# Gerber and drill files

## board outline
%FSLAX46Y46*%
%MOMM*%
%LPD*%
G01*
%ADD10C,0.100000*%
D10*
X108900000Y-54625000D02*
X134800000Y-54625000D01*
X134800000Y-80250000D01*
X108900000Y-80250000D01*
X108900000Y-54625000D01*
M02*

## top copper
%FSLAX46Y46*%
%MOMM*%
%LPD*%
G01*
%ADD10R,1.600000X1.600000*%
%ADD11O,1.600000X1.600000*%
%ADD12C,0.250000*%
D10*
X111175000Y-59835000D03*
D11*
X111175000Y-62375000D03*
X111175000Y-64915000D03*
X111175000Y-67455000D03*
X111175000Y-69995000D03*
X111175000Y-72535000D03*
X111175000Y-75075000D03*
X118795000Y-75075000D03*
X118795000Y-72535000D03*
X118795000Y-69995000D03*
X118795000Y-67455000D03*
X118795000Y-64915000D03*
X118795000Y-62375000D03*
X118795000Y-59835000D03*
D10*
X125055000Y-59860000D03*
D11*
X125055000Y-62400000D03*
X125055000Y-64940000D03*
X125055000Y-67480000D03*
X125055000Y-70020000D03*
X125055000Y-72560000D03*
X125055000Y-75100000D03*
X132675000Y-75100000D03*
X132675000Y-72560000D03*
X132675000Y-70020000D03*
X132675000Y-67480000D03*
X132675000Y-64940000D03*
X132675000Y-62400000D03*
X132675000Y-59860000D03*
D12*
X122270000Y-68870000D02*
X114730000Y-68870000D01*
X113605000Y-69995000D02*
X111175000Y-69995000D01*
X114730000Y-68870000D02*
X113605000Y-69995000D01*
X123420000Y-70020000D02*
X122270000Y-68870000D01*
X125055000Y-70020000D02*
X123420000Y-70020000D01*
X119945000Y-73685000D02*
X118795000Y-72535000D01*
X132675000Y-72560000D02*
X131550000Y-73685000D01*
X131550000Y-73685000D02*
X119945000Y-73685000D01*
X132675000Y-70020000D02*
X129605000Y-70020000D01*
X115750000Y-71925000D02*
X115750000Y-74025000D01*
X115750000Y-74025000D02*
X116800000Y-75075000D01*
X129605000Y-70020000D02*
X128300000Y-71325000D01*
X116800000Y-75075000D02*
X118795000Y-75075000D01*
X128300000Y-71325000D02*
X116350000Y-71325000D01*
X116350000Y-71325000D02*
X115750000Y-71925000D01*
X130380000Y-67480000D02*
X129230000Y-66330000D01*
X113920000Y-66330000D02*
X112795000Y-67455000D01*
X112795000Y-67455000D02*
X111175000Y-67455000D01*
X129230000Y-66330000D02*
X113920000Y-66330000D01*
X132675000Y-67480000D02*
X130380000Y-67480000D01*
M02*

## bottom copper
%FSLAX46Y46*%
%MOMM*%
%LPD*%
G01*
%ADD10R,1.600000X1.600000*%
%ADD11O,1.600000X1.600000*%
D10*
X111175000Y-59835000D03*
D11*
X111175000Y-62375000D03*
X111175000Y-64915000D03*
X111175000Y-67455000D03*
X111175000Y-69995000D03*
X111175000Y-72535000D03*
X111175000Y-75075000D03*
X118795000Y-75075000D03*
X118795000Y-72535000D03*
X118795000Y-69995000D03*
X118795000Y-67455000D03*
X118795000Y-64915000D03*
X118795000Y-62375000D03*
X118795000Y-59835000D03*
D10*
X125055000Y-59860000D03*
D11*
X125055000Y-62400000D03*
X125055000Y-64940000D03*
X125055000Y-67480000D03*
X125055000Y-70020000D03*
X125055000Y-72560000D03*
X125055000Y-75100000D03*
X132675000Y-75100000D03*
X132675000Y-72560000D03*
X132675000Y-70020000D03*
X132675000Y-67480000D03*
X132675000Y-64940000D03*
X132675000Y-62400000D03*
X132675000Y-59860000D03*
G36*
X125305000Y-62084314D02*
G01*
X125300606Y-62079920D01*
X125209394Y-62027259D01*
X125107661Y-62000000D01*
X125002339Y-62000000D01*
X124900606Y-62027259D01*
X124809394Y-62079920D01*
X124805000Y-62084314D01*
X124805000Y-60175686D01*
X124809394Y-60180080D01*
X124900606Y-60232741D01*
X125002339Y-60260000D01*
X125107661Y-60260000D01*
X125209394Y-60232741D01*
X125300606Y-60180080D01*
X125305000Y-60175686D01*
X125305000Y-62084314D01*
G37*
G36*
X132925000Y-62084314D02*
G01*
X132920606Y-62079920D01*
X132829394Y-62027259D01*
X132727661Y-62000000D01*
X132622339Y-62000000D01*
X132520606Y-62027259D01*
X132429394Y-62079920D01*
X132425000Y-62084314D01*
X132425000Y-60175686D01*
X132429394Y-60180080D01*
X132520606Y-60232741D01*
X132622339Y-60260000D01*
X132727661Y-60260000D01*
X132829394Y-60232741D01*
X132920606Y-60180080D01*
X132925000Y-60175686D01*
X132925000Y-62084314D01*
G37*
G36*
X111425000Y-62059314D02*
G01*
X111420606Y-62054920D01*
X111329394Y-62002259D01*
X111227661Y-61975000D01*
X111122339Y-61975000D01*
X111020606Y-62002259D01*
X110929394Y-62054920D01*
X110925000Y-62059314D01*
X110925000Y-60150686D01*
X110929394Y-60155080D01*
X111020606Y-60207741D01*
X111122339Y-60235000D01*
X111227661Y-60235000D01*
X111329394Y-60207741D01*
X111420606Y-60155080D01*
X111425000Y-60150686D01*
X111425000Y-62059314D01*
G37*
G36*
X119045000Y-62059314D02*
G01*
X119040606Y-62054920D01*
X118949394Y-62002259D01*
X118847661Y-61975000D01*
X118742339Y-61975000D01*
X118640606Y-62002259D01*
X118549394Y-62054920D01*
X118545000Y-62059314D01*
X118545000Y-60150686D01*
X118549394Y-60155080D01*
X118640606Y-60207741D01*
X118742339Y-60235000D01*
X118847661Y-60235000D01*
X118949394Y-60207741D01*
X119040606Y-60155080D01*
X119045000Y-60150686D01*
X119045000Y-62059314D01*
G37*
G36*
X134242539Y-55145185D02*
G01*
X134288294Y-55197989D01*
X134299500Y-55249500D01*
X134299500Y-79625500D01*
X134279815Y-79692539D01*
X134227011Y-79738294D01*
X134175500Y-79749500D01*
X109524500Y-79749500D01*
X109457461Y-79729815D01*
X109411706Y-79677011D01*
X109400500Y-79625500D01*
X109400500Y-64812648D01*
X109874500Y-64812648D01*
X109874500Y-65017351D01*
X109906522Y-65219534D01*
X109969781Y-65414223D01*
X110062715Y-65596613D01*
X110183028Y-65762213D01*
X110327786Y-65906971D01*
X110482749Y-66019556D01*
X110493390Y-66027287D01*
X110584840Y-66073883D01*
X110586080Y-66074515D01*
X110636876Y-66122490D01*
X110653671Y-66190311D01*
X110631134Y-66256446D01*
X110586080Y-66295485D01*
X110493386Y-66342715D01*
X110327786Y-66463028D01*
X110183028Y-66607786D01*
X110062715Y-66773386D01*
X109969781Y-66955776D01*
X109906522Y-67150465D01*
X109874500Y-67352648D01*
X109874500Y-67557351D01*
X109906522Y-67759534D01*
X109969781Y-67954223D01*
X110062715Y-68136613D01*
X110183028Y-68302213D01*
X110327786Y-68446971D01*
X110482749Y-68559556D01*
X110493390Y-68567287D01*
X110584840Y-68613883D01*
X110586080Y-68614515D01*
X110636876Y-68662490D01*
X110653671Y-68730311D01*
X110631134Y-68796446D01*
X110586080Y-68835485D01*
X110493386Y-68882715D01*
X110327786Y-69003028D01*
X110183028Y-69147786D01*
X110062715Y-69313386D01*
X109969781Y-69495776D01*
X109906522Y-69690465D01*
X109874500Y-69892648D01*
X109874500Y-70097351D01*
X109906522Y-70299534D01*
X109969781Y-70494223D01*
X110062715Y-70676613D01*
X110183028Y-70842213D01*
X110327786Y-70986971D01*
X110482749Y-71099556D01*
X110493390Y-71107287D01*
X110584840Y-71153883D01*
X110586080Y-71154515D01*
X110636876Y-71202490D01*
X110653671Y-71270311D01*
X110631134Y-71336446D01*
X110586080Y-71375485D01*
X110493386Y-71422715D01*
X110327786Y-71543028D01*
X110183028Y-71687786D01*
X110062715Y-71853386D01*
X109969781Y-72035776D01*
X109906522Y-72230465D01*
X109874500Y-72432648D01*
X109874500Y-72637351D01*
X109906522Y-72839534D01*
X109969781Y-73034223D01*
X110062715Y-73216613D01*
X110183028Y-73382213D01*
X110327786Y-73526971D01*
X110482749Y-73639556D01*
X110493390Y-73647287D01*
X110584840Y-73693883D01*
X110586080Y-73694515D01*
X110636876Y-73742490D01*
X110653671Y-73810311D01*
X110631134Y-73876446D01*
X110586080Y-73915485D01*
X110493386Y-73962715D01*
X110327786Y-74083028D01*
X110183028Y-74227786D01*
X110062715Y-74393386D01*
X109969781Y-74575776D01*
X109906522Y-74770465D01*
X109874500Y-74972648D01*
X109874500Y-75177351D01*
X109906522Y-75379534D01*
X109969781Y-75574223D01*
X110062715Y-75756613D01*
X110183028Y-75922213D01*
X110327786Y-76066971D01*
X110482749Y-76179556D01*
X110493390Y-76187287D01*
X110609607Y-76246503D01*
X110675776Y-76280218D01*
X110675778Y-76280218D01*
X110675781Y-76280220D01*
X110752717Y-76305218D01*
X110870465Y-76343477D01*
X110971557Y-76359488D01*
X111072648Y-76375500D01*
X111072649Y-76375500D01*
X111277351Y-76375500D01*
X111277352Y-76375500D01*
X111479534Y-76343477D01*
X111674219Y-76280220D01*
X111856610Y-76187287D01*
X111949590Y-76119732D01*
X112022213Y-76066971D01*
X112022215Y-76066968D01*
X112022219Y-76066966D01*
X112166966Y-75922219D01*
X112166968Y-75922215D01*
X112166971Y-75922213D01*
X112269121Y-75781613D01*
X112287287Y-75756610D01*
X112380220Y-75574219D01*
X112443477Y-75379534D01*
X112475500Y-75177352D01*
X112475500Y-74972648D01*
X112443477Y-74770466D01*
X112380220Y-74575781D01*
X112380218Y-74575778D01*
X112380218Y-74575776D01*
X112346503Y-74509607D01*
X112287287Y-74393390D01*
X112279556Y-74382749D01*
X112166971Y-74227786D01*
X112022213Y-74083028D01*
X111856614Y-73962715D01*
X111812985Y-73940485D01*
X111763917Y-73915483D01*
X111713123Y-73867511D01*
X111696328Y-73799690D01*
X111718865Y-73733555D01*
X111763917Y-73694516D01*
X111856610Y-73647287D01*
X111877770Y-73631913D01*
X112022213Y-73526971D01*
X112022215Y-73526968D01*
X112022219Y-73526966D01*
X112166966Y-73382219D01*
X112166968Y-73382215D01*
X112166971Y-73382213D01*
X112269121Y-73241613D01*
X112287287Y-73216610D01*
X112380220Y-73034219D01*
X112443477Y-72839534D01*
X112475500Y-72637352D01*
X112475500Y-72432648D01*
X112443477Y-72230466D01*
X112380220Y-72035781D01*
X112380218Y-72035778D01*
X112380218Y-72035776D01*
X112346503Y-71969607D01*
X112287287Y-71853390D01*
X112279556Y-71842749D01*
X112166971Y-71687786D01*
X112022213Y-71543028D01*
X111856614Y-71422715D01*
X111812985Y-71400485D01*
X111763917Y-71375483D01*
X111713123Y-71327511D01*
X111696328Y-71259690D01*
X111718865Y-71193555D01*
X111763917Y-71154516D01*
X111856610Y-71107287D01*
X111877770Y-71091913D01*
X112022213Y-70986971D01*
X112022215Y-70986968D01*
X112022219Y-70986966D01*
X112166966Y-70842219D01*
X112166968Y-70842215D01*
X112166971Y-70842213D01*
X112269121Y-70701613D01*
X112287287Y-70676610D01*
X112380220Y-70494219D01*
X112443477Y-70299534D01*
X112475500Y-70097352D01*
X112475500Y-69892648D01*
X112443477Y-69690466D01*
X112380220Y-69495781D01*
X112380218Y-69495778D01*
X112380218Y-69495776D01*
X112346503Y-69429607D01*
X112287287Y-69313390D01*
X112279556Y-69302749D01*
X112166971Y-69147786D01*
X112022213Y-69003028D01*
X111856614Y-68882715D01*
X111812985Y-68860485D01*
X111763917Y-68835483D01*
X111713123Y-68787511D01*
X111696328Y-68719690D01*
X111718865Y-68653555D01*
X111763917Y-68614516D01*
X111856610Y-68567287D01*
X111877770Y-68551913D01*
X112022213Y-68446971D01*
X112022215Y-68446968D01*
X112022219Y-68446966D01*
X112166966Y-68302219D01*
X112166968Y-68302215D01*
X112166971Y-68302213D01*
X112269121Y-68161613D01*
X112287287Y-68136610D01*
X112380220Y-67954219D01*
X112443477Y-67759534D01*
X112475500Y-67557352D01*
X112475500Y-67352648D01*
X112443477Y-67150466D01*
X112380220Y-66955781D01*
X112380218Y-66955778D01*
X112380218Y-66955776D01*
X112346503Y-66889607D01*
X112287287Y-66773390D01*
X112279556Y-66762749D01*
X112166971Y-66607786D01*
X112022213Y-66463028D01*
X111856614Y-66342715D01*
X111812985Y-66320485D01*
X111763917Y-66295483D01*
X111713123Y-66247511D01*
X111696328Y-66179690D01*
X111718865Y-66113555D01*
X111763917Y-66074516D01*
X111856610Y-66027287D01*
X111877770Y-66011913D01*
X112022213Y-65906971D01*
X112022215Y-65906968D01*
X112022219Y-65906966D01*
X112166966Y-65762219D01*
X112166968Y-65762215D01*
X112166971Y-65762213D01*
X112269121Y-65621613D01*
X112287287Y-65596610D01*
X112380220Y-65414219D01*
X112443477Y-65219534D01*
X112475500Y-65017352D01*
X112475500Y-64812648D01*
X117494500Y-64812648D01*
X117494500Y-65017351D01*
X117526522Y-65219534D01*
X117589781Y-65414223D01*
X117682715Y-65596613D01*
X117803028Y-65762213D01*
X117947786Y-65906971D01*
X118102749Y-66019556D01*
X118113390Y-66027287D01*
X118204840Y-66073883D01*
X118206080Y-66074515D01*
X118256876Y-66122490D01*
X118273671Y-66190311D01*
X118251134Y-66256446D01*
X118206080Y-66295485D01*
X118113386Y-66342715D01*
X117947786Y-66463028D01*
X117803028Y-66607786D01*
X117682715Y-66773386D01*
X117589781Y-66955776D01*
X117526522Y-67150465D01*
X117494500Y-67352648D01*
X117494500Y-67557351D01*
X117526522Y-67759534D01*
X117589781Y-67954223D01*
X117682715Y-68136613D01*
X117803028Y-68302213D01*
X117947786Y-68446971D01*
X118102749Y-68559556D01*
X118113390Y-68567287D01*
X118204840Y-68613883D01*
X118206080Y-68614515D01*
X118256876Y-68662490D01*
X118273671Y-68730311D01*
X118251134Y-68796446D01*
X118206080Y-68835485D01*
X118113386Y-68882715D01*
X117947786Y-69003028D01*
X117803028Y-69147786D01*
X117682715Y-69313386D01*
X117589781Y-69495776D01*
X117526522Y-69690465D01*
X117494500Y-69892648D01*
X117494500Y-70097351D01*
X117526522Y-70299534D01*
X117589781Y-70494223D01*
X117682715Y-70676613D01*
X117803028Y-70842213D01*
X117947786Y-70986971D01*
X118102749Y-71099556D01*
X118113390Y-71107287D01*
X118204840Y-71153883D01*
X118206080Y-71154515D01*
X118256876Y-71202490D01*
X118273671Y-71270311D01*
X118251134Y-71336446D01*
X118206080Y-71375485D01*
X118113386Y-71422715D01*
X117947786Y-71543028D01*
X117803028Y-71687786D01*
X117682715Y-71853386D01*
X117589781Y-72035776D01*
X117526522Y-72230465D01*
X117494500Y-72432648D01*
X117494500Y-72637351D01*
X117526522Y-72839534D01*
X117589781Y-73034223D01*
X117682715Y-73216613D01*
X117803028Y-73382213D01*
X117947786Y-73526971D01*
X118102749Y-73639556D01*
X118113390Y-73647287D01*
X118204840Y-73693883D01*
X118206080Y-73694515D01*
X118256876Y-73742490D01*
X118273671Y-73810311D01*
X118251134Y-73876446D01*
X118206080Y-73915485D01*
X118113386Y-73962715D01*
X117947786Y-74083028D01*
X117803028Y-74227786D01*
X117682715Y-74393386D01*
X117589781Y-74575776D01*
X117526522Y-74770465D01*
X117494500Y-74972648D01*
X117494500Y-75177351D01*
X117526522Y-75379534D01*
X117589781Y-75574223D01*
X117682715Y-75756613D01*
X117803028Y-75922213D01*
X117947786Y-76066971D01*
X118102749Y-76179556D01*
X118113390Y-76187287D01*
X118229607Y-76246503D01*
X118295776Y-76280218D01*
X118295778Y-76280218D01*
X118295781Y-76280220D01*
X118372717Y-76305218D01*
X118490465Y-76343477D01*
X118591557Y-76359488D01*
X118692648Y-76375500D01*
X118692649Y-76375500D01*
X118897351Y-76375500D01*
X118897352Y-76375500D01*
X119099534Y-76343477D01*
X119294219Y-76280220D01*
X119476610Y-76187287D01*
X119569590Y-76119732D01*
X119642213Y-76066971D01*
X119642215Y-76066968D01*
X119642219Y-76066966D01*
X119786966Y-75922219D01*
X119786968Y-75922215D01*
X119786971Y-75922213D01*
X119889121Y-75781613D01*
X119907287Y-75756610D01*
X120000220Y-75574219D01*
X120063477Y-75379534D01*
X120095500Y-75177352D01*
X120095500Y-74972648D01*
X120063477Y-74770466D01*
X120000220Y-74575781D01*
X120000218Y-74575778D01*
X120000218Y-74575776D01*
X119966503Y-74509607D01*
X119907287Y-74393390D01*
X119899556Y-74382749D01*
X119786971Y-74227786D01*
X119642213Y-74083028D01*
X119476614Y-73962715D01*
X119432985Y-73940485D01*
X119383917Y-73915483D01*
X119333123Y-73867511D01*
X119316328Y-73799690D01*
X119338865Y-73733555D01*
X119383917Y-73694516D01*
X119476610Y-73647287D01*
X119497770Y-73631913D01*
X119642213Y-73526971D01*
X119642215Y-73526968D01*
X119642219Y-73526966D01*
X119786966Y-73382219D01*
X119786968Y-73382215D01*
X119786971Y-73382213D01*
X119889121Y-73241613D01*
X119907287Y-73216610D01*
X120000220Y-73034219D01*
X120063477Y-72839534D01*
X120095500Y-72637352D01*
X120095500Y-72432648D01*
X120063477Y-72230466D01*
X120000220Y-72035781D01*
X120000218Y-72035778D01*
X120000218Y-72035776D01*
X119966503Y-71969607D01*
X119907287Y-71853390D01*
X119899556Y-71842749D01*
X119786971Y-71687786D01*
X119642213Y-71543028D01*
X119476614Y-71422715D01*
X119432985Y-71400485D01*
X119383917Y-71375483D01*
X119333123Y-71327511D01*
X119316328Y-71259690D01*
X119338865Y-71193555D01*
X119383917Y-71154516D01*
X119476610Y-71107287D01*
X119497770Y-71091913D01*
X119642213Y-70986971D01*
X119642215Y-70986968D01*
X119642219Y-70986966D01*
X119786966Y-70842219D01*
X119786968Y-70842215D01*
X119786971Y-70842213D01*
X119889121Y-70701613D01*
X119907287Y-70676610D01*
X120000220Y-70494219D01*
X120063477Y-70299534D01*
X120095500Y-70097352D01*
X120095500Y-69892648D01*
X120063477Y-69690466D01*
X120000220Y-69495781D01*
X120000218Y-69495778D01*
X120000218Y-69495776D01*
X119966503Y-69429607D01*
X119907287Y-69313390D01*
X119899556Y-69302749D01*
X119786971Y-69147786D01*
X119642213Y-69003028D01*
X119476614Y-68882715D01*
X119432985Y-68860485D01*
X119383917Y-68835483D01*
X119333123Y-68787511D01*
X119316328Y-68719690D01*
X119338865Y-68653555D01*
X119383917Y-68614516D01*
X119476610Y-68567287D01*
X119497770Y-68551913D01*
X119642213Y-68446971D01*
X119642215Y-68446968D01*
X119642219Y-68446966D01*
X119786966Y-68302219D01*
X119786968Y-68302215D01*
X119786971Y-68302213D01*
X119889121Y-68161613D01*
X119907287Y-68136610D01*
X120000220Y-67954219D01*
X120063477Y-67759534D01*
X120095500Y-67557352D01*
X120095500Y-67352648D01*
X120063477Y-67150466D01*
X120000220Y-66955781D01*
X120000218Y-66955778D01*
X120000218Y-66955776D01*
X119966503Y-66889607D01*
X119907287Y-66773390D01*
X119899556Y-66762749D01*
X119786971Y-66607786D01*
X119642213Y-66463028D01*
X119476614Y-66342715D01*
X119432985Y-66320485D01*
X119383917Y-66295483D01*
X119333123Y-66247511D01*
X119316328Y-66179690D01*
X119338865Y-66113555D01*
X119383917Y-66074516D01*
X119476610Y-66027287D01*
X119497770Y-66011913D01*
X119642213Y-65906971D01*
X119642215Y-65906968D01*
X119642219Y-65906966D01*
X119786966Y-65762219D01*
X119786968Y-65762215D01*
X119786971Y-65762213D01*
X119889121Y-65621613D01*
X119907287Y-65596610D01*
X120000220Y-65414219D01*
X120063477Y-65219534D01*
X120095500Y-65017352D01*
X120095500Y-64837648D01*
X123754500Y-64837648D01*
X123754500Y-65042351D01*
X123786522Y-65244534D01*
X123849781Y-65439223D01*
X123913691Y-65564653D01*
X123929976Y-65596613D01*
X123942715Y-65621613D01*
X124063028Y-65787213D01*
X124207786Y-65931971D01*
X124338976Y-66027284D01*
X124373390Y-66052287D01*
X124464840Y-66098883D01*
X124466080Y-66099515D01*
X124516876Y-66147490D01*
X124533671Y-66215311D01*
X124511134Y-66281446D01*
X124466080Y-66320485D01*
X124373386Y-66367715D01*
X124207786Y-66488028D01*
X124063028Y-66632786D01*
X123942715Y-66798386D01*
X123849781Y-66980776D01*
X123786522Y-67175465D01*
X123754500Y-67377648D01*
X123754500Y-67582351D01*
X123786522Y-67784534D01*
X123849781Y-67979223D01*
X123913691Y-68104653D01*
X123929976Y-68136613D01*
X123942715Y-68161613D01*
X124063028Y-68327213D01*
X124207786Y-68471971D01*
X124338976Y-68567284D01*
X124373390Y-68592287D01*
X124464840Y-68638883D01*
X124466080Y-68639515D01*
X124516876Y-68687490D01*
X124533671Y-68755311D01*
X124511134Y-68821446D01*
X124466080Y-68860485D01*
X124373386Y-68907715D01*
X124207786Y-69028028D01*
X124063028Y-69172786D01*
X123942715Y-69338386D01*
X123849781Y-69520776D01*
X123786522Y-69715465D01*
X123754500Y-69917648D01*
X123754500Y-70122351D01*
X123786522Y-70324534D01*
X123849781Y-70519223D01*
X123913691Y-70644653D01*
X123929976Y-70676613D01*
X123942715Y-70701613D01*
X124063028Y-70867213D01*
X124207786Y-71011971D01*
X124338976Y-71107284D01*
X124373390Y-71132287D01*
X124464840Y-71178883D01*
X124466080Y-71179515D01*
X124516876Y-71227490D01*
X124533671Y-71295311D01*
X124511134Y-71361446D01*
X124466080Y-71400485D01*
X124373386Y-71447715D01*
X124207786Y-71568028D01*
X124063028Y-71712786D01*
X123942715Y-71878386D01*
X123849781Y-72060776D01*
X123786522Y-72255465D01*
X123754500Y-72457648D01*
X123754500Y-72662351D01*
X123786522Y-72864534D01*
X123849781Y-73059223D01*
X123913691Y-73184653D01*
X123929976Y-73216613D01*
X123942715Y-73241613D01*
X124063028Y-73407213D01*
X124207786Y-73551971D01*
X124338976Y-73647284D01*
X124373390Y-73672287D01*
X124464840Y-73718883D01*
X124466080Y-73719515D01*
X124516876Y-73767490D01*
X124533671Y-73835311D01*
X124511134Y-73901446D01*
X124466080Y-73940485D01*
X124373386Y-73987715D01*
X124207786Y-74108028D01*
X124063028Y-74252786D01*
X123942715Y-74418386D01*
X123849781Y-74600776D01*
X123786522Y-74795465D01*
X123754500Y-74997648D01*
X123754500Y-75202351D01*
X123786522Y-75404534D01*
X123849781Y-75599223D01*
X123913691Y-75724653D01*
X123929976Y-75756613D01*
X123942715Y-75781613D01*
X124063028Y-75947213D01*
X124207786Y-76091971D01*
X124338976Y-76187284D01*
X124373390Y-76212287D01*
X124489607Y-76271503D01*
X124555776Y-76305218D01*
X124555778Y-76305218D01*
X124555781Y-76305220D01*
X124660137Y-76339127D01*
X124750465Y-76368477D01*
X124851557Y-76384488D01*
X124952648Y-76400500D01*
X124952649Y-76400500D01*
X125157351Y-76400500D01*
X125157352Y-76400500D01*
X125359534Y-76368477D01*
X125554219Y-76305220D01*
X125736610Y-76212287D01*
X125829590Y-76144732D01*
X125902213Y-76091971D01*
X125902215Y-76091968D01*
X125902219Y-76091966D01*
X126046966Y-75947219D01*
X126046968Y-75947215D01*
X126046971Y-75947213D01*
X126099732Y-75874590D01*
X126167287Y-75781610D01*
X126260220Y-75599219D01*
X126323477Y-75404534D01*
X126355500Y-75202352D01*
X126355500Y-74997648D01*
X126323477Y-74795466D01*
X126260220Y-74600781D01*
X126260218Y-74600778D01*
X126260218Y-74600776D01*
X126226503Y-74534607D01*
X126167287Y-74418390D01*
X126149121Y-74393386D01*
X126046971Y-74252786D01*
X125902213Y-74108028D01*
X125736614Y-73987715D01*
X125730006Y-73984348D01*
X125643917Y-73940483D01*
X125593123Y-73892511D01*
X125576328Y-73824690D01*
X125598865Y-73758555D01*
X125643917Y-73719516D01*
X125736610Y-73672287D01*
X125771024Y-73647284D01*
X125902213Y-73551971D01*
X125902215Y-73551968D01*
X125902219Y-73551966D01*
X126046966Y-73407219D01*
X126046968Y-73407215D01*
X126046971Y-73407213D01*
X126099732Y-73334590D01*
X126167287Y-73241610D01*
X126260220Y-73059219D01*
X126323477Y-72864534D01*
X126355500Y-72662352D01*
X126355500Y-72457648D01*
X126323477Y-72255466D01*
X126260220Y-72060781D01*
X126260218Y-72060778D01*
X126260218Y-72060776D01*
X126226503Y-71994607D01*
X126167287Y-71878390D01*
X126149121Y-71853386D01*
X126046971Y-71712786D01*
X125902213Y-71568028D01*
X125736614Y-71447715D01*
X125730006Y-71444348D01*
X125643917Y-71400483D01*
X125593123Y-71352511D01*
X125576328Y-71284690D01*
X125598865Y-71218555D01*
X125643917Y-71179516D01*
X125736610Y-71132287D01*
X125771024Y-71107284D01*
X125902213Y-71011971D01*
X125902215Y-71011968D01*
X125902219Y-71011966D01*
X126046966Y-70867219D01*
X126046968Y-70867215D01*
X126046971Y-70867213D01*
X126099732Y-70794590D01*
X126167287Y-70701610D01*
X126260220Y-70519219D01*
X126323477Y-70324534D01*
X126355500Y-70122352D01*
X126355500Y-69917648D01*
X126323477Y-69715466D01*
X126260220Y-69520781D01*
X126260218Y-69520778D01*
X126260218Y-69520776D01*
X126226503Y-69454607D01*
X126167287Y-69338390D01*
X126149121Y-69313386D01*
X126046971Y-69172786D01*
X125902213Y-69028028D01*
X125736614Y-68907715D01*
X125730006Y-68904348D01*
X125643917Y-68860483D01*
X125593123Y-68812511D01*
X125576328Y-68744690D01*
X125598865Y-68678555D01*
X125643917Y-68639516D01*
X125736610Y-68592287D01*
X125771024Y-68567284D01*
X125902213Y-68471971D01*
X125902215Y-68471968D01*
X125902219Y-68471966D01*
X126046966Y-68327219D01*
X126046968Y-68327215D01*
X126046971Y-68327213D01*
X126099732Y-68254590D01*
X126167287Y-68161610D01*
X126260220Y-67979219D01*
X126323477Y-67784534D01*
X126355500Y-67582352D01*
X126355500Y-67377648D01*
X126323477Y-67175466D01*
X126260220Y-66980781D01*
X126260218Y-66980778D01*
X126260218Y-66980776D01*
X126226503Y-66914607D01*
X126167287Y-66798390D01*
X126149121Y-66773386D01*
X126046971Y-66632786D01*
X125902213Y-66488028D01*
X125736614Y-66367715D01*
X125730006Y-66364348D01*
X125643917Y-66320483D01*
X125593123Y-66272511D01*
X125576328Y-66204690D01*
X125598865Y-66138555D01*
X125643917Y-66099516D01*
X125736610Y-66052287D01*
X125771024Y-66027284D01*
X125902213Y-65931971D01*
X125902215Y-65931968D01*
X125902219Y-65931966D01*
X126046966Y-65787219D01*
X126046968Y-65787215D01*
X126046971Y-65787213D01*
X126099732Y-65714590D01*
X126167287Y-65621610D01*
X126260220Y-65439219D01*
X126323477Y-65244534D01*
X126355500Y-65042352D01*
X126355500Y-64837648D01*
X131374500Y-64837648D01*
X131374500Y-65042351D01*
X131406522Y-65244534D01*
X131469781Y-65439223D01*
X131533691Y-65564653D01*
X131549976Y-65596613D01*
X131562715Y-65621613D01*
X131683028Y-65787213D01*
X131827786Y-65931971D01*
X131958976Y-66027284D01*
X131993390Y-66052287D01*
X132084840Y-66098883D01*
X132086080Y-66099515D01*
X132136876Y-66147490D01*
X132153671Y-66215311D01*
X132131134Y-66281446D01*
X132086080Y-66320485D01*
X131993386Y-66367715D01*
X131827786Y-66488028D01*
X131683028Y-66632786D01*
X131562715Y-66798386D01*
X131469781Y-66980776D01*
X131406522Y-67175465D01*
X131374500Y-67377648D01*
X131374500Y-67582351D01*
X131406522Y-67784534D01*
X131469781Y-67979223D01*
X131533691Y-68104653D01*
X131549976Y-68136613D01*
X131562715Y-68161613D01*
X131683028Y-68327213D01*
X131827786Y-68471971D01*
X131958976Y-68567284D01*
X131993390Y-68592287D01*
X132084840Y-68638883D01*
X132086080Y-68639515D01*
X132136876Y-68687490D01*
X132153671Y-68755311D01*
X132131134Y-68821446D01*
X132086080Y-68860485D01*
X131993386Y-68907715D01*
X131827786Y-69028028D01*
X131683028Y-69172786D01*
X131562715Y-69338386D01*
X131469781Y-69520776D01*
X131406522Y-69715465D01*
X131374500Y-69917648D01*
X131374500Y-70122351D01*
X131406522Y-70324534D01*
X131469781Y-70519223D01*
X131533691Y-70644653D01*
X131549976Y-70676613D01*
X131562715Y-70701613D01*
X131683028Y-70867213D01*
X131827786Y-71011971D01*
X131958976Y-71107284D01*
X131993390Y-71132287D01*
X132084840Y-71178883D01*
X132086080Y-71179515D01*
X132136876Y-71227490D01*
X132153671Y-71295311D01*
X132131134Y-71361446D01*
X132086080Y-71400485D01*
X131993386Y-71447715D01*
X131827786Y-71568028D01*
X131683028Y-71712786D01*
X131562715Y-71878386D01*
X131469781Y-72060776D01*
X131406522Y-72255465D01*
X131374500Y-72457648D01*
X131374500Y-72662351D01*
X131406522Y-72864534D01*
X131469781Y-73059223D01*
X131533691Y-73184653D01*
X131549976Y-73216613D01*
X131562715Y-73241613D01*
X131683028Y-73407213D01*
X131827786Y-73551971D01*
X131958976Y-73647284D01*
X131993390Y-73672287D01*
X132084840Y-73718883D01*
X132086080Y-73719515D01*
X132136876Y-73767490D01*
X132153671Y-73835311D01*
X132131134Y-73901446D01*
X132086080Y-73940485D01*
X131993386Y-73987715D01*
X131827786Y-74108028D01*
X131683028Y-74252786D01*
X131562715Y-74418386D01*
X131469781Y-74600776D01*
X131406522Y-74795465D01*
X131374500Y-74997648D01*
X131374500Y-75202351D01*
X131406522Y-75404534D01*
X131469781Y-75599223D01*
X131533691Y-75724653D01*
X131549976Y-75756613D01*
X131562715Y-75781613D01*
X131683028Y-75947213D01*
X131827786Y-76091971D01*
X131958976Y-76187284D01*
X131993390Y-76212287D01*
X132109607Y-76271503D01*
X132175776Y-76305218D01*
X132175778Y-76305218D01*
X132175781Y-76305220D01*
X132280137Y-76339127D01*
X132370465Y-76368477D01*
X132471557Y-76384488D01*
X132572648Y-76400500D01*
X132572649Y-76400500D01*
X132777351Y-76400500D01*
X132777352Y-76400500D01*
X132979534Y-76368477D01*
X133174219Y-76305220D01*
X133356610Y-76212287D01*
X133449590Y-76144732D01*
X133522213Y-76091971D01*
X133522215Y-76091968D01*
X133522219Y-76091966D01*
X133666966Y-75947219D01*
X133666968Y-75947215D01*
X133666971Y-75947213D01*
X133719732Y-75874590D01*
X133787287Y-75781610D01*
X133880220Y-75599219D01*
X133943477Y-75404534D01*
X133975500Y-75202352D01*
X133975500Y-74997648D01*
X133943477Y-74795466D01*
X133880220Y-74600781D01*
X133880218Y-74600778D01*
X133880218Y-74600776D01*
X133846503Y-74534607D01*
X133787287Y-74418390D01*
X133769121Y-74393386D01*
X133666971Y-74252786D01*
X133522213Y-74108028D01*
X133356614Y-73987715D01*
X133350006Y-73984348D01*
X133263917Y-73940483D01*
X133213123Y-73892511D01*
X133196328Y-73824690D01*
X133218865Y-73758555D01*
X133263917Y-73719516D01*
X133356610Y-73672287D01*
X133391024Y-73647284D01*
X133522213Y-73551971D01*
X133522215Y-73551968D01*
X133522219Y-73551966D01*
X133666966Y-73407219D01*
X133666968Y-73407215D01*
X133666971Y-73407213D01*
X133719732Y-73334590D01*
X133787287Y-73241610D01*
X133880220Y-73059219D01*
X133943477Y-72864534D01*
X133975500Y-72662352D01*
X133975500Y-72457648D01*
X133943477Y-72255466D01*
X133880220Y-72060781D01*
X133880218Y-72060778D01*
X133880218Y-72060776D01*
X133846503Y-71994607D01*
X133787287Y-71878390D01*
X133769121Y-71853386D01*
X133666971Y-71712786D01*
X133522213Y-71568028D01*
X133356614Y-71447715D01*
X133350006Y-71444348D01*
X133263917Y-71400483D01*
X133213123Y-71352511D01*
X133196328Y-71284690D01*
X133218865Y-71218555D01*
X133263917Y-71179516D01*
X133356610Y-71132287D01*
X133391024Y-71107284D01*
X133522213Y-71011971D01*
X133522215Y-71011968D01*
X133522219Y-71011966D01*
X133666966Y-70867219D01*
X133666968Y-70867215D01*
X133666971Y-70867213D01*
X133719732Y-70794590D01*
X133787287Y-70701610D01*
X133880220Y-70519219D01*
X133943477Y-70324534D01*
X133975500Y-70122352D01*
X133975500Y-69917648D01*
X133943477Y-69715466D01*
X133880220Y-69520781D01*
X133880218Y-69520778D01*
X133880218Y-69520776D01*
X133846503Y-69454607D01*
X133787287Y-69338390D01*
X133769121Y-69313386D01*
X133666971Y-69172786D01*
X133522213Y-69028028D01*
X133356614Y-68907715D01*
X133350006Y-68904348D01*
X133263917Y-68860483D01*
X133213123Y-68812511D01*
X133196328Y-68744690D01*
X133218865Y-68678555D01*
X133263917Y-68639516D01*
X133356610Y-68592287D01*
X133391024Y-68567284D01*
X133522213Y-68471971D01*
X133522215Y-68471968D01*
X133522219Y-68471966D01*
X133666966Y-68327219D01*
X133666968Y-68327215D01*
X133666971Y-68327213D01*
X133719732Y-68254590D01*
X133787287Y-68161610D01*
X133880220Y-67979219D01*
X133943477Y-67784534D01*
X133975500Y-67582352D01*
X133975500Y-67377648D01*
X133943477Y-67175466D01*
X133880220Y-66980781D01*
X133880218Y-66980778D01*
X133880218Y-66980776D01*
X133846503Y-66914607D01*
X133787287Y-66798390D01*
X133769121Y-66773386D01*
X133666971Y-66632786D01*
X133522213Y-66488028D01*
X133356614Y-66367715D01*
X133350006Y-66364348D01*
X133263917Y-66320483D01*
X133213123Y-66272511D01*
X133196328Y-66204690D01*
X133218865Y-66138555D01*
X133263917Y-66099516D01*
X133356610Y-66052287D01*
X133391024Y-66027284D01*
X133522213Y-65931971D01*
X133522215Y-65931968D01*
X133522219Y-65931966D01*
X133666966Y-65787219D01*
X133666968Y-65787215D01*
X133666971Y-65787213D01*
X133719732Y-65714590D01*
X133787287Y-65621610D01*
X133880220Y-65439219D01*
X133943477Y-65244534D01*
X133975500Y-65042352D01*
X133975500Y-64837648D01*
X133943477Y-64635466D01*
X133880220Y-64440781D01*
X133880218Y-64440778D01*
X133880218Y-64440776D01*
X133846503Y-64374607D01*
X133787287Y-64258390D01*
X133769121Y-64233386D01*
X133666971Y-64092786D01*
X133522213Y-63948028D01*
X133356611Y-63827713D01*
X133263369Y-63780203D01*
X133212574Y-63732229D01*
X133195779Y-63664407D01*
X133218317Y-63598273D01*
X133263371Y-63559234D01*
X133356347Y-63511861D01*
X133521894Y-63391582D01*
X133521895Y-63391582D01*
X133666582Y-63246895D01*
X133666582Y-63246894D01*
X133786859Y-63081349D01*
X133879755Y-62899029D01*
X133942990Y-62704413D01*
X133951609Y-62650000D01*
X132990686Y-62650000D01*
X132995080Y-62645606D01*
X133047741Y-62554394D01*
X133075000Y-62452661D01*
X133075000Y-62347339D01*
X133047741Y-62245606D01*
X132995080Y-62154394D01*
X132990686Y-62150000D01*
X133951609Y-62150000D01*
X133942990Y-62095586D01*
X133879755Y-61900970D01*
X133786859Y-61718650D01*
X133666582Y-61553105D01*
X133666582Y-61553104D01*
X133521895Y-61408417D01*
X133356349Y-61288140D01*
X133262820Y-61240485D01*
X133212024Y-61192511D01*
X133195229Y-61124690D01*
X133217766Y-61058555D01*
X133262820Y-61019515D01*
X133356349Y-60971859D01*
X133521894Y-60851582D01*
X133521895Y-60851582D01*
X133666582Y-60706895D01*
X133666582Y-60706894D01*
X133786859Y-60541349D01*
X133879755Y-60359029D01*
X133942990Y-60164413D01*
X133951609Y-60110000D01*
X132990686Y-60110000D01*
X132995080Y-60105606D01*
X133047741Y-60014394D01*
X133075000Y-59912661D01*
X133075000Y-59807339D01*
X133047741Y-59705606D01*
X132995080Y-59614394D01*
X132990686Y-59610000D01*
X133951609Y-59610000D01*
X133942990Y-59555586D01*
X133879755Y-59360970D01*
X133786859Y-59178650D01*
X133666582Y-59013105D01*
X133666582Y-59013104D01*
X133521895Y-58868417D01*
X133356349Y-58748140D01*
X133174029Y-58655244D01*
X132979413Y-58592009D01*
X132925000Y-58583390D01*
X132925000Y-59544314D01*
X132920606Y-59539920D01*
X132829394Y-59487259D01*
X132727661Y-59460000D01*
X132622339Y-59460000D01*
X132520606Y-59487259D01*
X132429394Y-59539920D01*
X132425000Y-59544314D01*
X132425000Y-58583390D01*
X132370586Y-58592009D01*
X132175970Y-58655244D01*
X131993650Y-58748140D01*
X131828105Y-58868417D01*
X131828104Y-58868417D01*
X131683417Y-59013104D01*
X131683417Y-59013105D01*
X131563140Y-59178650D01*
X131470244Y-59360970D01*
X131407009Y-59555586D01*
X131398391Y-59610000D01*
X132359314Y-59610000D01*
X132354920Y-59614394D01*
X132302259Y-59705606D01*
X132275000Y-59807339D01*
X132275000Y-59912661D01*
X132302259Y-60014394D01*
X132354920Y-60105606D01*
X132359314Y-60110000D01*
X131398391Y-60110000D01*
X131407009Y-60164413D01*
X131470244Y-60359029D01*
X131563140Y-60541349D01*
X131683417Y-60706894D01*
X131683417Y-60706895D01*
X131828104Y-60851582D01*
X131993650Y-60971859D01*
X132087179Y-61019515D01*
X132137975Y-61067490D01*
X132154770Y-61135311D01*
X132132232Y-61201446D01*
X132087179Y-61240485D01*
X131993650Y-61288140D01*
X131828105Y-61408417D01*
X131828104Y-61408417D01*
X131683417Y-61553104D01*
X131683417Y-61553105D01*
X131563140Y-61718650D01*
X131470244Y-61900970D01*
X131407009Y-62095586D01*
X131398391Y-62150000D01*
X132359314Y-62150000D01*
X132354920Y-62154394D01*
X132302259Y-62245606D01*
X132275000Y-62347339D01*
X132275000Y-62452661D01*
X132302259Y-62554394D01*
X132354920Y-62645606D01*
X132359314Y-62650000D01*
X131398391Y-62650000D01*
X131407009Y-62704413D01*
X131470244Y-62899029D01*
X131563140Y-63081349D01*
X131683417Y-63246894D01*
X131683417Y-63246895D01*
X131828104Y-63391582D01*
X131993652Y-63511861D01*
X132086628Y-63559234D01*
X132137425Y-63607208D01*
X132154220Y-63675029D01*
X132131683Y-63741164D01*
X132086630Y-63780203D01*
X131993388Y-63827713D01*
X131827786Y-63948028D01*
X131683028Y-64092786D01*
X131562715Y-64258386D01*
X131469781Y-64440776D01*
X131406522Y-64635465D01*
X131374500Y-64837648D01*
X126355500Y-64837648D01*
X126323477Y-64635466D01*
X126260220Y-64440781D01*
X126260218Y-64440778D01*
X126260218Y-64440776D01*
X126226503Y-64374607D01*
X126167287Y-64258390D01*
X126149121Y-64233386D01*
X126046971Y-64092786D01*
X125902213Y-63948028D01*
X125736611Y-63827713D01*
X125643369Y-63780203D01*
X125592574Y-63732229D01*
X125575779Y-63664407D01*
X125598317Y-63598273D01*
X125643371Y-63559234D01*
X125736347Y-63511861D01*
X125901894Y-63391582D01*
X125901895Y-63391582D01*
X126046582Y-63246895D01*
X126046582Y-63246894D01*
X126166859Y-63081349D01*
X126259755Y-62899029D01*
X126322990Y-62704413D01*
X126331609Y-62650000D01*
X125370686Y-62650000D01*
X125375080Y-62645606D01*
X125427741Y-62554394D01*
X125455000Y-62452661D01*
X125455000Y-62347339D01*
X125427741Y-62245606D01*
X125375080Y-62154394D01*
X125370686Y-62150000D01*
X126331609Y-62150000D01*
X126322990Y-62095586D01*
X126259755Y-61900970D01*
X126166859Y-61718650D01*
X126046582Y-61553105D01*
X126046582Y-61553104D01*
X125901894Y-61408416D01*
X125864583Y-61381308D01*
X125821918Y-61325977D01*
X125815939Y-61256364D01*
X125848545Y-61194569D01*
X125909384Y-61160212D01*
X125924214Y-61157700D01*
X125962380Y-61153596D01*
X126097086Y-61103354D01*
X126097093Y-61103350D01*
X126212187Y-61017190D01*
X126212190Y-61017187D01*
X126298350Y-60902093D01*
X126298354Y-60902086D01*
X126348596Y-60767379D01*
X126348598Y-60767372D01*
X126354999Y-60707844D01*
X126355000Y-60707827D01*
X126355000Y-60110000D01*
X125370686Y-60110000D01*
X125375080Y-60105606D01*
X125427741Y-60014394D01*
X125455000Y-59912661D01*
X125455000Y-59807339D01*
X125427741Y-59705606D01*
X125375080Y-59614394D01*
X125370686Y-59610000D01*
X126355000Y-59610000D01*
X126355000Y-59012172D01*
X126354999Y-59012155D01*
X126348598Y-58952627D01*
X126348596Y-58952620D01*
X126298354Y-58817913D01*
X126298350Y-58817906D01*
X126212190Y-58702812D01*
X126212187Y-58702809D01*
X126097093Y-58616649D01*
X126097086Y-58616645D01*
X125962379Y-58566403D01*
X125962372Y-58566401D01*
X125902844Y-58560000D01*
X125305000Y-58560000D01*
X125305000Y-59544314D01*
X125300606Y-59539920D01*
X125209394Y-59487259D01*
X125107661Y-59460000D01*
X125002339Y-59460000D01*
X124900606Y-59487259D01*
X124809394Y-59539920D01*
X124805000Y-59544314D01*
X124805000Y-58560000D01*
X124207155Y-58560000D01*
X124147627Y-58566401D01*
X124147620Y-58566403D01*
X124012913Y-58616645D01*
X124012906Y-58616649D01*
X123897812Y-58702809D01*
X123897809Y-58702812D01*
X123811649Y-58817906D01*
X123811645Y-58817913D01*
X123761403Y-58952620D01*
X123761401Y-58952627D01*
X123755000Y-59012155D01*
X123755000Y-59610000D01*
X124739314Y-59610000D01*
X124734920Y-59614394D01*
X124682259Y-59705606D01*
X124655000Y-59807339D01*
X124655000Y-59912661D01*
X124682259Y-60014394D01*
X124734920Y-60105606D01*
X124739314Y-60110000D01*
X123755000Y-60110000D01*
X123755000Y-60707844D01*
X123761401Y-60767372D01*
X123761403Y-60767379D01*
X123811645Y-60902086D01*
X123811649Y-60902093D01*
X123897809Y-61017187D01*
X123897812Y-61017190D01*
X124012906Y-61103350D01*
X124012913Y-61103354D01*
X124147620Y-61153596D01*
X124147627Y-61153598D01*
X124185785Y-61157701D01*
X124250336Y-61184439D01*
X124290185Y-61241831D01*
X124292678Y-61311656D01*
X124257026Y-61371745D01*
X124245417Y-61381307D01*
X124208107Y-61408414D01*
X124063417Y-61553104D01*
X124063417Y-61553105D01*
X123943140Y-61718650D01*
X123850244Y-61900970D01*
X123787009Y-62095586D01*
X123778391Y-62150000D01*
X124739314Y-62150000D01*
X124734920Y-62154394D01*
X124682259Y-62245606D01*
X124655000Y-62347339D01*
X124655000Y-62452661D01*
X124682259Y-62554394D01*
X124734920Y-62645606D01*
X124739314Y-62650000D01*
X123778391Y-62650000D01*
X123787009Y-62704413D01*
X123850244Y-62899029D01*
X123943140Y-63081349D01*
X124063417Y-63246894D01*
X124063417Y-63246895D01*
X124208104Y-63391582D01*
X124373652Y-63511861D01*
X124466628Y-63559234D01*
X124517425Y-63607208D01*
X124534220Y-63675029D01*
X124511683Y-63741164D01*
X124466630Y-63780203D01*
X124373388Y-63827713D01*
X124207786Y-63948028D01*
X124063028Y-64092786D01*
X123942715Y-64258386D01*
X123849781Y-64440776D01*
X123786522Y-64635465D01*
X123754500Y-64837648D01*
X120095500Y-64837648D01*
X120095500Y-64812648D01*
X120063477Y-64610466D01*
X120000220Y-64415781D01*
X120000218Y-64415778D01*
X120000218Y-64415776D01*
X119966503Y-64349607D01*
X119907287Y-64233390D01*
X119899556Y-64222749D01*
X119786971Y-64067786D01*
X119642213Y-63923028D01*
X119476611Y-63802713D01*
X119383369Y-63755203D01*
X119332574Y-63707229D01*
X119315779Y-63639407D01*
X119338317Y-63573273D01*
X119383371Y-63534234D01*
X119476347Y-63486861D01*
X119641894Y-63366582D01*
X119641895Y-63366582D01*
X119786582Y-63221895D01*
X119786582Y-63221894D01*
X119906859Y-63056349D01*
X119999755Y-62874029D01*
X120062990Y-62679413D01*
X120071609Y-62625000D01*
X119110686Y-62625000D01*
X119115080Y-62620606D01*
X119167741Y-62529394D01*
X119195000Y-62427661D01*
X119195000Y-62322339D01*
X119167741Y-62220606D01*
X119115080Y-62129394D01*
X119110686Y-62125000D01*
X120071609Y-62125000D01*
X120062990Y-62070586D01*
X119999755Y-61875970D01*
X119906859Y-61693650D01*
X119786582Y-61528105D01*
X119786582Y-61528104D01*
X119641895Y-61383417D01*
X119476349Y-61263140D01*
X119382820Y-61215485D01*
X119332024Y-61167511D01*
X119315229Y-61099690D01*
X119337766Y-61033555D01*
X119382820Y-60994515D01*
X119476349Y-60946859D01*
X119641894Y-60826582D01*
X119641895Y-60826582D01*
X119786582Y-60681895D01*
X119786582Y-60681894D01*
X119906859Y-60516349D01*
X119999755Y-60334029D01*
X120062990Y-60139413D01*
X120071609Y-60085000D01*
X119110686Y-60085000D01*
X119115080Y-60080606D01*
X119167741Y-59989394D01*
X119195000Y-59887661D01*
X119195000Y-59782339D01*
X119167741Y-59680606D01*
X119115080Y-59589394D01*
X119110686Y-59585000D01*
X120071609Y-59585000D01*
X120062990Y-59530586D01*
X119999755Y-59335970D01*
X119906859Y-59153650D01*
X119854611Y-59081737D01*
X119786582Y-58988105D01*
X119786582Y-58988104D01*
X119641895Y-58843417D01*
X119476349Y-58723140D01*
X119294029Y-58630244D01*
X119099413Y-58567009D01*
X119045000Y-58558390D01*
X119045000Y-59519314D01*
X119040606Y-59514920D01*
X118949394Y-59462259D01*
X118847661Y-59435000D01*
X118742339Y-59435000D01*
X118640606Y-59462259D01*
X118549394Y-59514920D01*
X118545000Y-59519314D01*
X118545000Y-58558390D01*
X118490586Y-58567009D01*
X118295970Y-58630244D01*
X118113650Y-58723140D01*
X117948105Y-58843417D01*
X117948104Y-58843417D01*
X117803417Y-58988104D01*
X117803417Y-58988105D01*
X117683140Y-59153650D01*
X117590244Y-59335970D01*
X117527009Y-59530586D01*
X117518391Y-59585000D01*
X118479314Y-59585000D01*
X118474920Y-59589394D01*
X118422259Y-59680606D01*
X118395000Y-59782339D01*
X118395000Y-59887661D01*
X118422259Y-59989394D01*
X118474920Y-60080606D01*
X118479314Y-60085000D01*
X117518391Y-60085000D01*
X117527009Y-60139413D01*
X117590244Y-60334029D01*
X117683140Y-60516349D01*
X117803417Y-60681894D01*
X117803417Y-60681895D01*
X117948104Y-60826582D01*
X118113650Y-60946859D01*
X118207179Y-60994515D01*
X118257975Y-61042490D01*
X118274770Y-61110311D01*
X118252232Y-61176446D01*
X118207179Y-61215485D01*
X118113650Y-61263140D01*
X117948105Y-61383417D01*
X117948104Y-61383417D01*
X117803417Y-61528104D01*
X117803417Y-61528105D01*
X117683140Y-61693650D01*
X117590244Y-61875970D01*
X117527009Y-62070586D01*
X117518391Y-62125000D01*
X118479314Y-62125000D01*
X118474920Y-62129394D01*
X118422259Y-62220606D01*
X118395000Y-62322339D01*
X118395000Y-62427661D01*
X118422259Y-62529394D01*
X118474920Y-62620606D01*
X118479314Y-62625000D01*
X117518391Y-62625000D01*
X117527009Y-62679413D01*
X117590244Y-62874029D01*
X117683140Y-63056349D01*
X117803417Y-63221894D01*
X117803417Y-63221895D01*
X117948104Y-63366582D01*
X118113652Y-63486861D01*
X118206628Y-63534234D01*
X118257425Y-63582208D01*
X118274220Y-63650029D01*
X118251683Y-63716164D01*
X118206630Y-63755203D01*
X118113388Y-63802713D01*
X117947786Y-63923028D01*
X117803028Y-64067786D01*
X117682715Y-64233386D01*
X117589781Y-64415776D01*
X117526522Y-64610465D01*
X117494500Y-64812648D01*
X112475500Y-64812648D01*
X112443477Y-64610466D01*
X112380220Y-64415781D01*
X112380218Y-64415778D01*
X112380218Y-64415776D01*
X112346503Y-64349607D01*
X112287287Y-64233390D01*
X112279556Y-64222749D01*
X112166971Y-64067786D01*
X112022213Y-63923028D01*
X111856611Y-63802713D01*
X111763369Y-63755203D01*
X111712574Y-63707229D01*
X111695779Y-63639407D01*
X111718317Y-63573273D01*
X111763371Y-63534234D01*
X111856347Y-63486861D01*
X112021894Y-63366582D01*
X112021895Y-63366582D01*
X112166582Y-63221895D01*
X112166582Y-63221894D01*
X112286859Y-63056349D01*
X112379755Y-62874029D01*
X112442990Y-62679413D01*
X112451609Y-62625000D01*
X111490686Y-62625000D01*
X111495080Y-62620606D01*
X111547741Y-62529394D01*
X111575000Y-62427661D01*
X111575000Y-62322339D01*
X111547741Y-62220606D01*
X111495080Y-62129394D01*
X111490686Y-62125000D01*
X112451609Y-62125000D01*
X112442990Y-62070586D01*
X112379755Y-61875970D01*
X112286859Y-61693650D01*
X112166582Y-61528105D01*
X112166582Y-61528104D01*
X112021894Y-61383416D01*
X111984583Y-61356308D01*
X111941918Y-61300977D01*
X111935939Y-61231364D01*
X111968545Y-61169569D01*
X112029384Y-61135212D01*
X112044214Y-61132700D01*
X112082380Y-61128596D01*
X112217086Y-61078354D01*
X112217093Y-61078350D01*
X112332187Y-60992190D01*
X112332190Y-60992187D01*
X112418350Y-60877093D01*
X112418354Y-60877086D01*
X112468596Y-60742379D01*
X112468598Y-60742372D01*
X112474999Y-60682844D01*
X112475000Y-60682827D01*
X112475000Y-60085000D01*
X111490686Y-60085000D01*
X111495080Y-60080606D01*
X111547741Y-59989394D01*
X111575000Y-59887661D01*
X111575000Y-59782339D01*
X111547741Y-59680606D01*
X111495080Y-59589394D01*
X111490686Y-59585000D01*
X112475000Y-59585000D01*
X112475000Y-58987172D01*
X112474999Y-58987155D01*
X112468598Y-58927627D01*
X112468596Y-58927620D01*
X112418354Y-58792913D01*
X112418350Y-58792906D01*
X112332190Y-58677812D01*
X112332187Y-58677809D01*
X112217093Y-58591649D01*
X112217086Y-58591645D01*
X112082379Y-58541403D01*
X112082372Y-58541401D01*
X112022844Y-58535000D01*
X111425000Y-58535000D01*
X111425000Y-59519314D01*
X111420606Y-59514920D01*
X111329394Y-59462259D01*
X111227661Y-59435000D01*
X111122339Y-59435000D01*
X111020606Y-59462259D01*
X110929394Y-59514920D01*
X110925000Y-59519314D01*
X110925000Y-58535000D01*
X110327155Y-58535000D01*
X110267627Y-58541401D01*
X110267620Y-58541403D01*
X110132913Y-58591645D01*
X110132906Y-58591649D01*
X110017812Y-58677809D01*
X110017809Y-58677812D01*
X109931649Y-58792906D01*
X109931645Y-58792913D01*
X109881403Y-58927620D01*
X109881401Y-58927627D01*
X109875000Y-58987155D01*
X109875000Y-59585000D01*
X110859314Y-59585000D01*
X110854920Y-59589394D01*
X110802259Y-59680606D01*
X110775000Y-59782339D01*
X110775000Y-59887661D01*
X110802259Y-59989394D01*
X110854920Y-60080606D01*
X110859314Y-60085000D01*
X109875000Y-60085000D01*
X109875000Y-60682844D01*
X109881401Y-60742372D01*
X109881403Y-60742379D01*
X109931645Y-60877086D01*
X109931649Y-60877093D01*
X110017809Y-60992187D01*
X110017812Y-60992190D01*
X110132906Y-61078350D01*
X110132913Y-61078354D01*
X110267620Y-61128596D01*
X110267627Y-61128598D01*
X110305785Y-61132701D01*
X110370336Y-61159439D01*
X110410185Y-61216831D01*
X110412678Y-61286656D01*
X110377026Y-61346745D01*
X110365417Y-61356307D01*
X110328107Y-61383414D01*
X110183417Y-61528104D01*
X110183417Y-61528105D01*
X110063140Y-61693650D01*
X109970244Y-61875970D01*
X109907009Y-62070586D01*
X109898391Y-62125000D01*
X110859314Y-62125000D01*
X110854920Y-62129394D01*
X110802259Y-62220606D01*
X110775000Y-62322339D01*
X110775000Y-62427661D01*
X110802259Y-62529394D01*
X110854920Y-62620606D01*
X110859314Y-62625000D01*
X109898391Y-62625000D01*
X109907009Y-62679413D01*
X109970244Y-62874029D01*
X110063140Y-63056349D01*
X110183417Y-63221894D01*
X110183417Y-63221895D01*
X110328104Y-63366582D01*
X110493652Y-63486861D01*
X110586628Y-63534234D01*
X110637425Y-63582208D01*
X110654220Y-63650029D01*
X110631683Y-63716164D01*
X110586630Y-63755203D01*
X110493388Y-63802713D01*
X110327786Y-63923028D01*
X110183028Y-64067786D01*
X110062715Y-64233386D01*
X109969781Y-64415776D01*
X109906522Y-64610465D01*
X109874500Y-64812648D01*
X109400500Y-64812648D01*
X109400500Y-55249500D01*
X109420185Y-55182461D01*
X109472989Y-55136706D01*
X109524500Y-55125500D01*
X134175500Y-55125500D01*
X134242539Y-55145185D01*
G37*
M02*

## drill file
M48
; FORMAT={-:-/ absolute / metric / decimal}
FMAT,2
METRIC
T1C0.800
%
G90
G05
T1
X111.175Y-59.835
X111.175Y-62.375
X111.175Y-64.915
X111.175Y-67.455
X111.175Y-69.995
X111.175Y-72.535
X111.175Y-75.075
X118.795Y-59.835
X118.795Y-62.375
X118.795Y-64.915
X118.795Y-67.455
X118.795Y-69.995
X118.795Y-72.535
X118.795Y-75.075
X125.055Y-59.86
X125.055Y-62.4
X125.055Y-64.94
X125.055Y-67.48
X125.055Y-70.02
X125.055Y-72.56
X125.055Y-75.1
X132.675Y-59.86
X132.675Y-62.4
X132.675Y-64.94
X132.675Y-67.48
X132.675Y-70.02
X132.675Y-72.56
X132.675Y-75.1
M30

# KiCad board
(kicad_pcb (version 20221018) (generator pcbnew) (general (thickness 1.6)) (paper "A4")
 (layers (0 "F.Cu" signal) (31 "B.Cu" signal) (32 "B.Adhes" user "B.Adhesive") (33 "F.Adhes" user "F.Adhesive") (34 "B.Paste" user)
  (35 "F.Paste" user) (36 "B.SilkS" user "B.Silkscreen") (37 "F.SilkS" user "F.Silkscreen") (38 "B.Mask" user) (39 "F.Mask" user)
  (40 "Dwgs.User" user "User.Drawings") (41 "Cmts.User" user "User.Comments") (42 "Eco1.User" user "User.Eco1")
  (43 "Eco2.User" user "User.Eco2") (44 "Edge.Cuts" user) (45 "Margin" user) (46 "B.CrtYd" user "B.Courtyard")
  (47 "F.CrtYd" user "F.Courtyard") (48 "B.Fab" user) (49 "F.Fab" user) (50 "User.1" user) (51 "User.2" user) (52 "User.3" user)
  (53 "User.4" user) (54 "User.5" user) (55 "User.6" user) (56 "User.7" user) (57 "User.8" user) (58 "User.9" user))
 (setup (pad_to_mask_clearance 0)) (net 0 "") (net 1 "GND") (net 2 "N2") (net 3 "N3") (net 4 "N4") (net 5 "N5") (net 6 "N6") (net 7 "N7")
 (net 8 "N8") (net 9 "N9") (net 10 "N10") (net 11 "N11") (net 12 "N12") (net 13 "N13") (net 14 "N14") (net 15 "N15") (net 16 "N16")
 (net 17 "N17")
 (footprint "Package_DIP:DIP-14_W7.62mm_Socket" (layer "F.Cu") (at 111.175 59.835)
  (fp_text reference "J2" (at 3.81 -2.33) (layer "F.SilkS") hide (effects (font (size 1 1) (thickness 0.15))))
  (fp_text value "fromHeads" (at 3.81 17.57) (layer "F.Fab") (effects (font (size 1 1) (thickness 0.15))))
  (pad "1" thru_hole rect (at 0 0) (size 1.6 1.6) (drill 0.8) (layers "*.Cu" "*.Mask") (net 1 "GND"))
  (pad "2" thru_hole oval (at 0 2.54) (size 1.6 1.6) (drill 0.8) (layers "*.Cu" "*.Mask") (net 1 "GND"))
  (pad "3" thru_hole oval (at 0 5.08) (size 1.6 1.6) (drill 0.8) (layers "*.Cu" "*.Mask") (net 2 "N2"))
  (pad "4" thru_hole oval (at 0 7.62) (size 1.6 1.6) (drill 0.8) (layers "*.Cu" "*.Mask") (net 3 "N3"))
  (pad "5" thru_hole oval (at 0 10.16) (size 1.6 1.6) (drill 0.8) (layers "*.Cu" "*.Mask") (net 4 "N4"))
  (pad "6" thru_hole oval (at 0 12.7) (size 1.6 1.6) (drill 0.8) (layers "*.Cu" "*.Mask") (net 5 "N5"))
  (pad "7" thru_hole oval (at 0 15.24) (size 1.6 1.6) (drill 0.8) (layers "*.Cu" "*.Mask") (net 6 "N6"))
  (pad "8" thru_hole oval (at 7.62 15.24) (size 1.6 1.6) (drill 0.8) (layers "*.Cu" "*.Mask") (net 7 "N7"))
  (pad "9" thru_hole oval (at 7.62 12.7) (size 1.6 1.6) (drill 0.8) (layers "*.Cu" "*.Mask") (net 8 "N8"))
  (pad "10" thru_hole oval (at 7.62 10.16) (size 1.6 1.6) (drill 0.8) (layers "*.Cu" "*.Mask") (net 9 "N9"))
  (pad "11" thru_hole oval (at 7.62 7.62) (size 1.6 1.6) (drill 0.8) (layers "*.Cu" "*.Mask") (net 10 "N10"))
  (pad "12" thru_hole oval (at 7.62 5.08) (size 1.6 1.6) (drill 0.8) (layers "*.Cu" "*.Mask") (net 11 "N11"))
  (pad "13" thru_hole oval (at 7.62 2.54) (size 1.6 1.6) (drill 0.8) (layers "*.Cu" "*.Mask") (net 1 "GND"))
  (pad "14" thru_hole oval (at 7.62 0) (size 1.6 1.6) (drill 0.8) (layers "*.Cu" "*.Mask") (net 1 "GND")))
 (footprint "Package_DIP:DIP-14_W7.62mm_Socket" (layer "F.Cu") (at 125.055 59.86)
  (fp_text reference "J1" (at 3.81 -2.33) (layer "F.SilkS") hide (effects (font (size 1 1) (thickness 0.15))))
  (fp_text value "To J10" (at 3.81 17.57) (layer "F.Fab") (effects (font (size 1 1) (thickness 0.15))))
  (pad "1" thru_hole rect (at 0 0) (size 1.6 1.6) (drill 0.8) (layers "*.Cu" "*.Mask") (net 1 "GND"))
  (pad "2" thru_hole oval (at 0 2.54) (size 1.6 1.6) (drill 0.8) (layers "*.Cu" "*.Mask") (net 1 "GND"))
  (pad "3" thru_hole oval (at 0 5.08) (size 1.6 1.6) (drill 0.8) (layers "*.Cu" "*.Mask") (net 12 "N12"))
  (pad "4" thru_hole oval (at 0 7.62) (size 1.6 1.6) (drill 0.8) (layers "*.Cu" "*.Mask") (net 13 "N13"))
  (pad "5" thru_hole oval (at 0 10.16) (size 1.6 1.6) (drill 0.8) (layers "*.Cu" "*.Mask") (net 4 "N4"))
  (pad "6" thru_hole oval (at 0 12.7) (size 1.6 1.6) (drill 0.8) (layers "*.Cu" "*.Mask") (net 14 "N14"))
  (pad "7" thru_hole oval (at 0 15.24) (size 1.6 1.6) (drill 0.8) (layers "*.Cu" "*.Mask") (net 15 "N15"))
  (pad "8" thru_hole oval (at 7.62 15.24) (size 1.6 1.6) (drill 0.8) (layers "*.Cu" "*.Mask") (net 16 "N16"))
  (pad "9" thru_hole oval (at 7.62 12.7) (size 1.6 1.6) (drill 0.8) (layers "*.Cu" "*.Mask") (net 8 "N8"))
  (pad "10" thru_hole oval (at 7.62 10.16) (size 1.6 1.6) (drill 0.8) (layers "*.Cu" "*.Mask") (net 7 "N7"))
  (pad "11" thru_hole oval (at 7.62 7.62) (size 1.6 1.6) (drill 0.8) (layers "*.Cu" "*.Mask") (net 3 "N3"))
  (pad "12" thru_hole oval (at 7.62 5.08) (size 1.6 1.6) (drill 0.8) (layers "*.Cu" "*.Mask") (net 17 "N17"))
  (pad "13" thru_hole oval (at 7.62 2.54) (size 1.6 1.6) (drill 0.8) (layers "*.Cu" "*.Mask") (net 1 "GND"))
  (pad "14" thru_hole oval (at 7.62 0) (size 1.6 1.6) (drill 0.8) (layers "*.Cu" "*.Mask") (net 1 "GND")))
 (gr_rect (start 108.9 54.625) (end 134.8 80.25) (stroke (width 0.1) (type default)) (fill none) (layer "Edge.Cuts"))
 (segment (start 122.27 68.87) (end 114.73 68.87) (width 0.25) (layer "F.Cu") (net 4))
 (segment (start 113.605 69.995) (end 111.175 69.995) (width 0.25) (layer "F.Cu") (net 4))
 (segment (start 114.73 68.87) (end 113.605 69.995) (width 0.25) (layer "F.Cu") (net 4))
 (segment (start 123.42 70.02) (end 122.27 68.87) (width 0.25) (layer "F.Cu") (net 4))
 (segment (start 125.055 70.02) (end 123.42 70.02) (width 0.25) (layer "F.Cu") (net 4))
 (segment (start 119.945 73.685) (end 118.795 72.535) (width 0.25) (layer "F.Cu") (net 8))
 (segment (start 132.675 72.56) (end 131.55 73.685) (width 0.25) (layer "F.Cu") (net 8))
 (segment (start 131.55 73.685) (end 119.945 73.685) (width 0.25) (layer "F.Cu") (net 8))
 (segment (start 132.675 70.02) (end 129.605 70.02) (width 0.25) (layer "F.Cu") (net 7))
 (segment (start 115.75 71.925) (end 115.75 74.025) (width 0.25) (layer "F.Cu") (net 7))
 (segment (start 115.75 74.025) (end 116.8 75.075) (width 0.25) (layer "F.Cu") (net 7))
 (segment (start 129.605 70.02) (end 128.3 71.325) (width 0.25) (layer "F.Cu") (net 7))
 (segment (start 116.8 75.075) (end 118.795 75.075) (width 0.25) (layer "F.Cu") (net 7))
 (segment (start 128.3 71.325) (end 116.35 71.325) (width 0.25) (layer "F.Cu") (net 7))
 (segment (start 116.35 71.325) (end 115.75 71.925) (width 0.25) (layer "F.Cu") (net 7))
 (segment (start 130.38 67.48) (end 129.23 66.33) (width 0.25) (layer "F.Cu") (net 3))
 (segment (start 113.92 66.33) (end 112.795 67.455) (width 0.25) (layer "F.Cu") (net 3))
 (segment (start 112.795 67.455) (end 111.175 67.455) (width 0.25) (layer "F.Cu") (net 3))
 (segment (start 129.23 66.33) (end 113.92 66.33) (width 0.25) (layer "F.Cu") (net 3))
 (segment (start 132.675 67.48) (end 130.38 67.48) (width 0.25) (layer "F.Cu") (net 3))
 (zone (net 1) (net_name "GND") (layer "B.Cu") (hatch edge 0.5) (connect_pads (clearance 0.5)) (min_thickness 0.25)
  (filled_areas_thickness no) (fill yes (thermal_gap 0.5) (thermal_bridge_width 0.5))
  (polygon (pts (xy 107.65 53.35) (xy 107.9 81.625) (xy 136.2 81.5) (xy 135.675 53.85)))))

